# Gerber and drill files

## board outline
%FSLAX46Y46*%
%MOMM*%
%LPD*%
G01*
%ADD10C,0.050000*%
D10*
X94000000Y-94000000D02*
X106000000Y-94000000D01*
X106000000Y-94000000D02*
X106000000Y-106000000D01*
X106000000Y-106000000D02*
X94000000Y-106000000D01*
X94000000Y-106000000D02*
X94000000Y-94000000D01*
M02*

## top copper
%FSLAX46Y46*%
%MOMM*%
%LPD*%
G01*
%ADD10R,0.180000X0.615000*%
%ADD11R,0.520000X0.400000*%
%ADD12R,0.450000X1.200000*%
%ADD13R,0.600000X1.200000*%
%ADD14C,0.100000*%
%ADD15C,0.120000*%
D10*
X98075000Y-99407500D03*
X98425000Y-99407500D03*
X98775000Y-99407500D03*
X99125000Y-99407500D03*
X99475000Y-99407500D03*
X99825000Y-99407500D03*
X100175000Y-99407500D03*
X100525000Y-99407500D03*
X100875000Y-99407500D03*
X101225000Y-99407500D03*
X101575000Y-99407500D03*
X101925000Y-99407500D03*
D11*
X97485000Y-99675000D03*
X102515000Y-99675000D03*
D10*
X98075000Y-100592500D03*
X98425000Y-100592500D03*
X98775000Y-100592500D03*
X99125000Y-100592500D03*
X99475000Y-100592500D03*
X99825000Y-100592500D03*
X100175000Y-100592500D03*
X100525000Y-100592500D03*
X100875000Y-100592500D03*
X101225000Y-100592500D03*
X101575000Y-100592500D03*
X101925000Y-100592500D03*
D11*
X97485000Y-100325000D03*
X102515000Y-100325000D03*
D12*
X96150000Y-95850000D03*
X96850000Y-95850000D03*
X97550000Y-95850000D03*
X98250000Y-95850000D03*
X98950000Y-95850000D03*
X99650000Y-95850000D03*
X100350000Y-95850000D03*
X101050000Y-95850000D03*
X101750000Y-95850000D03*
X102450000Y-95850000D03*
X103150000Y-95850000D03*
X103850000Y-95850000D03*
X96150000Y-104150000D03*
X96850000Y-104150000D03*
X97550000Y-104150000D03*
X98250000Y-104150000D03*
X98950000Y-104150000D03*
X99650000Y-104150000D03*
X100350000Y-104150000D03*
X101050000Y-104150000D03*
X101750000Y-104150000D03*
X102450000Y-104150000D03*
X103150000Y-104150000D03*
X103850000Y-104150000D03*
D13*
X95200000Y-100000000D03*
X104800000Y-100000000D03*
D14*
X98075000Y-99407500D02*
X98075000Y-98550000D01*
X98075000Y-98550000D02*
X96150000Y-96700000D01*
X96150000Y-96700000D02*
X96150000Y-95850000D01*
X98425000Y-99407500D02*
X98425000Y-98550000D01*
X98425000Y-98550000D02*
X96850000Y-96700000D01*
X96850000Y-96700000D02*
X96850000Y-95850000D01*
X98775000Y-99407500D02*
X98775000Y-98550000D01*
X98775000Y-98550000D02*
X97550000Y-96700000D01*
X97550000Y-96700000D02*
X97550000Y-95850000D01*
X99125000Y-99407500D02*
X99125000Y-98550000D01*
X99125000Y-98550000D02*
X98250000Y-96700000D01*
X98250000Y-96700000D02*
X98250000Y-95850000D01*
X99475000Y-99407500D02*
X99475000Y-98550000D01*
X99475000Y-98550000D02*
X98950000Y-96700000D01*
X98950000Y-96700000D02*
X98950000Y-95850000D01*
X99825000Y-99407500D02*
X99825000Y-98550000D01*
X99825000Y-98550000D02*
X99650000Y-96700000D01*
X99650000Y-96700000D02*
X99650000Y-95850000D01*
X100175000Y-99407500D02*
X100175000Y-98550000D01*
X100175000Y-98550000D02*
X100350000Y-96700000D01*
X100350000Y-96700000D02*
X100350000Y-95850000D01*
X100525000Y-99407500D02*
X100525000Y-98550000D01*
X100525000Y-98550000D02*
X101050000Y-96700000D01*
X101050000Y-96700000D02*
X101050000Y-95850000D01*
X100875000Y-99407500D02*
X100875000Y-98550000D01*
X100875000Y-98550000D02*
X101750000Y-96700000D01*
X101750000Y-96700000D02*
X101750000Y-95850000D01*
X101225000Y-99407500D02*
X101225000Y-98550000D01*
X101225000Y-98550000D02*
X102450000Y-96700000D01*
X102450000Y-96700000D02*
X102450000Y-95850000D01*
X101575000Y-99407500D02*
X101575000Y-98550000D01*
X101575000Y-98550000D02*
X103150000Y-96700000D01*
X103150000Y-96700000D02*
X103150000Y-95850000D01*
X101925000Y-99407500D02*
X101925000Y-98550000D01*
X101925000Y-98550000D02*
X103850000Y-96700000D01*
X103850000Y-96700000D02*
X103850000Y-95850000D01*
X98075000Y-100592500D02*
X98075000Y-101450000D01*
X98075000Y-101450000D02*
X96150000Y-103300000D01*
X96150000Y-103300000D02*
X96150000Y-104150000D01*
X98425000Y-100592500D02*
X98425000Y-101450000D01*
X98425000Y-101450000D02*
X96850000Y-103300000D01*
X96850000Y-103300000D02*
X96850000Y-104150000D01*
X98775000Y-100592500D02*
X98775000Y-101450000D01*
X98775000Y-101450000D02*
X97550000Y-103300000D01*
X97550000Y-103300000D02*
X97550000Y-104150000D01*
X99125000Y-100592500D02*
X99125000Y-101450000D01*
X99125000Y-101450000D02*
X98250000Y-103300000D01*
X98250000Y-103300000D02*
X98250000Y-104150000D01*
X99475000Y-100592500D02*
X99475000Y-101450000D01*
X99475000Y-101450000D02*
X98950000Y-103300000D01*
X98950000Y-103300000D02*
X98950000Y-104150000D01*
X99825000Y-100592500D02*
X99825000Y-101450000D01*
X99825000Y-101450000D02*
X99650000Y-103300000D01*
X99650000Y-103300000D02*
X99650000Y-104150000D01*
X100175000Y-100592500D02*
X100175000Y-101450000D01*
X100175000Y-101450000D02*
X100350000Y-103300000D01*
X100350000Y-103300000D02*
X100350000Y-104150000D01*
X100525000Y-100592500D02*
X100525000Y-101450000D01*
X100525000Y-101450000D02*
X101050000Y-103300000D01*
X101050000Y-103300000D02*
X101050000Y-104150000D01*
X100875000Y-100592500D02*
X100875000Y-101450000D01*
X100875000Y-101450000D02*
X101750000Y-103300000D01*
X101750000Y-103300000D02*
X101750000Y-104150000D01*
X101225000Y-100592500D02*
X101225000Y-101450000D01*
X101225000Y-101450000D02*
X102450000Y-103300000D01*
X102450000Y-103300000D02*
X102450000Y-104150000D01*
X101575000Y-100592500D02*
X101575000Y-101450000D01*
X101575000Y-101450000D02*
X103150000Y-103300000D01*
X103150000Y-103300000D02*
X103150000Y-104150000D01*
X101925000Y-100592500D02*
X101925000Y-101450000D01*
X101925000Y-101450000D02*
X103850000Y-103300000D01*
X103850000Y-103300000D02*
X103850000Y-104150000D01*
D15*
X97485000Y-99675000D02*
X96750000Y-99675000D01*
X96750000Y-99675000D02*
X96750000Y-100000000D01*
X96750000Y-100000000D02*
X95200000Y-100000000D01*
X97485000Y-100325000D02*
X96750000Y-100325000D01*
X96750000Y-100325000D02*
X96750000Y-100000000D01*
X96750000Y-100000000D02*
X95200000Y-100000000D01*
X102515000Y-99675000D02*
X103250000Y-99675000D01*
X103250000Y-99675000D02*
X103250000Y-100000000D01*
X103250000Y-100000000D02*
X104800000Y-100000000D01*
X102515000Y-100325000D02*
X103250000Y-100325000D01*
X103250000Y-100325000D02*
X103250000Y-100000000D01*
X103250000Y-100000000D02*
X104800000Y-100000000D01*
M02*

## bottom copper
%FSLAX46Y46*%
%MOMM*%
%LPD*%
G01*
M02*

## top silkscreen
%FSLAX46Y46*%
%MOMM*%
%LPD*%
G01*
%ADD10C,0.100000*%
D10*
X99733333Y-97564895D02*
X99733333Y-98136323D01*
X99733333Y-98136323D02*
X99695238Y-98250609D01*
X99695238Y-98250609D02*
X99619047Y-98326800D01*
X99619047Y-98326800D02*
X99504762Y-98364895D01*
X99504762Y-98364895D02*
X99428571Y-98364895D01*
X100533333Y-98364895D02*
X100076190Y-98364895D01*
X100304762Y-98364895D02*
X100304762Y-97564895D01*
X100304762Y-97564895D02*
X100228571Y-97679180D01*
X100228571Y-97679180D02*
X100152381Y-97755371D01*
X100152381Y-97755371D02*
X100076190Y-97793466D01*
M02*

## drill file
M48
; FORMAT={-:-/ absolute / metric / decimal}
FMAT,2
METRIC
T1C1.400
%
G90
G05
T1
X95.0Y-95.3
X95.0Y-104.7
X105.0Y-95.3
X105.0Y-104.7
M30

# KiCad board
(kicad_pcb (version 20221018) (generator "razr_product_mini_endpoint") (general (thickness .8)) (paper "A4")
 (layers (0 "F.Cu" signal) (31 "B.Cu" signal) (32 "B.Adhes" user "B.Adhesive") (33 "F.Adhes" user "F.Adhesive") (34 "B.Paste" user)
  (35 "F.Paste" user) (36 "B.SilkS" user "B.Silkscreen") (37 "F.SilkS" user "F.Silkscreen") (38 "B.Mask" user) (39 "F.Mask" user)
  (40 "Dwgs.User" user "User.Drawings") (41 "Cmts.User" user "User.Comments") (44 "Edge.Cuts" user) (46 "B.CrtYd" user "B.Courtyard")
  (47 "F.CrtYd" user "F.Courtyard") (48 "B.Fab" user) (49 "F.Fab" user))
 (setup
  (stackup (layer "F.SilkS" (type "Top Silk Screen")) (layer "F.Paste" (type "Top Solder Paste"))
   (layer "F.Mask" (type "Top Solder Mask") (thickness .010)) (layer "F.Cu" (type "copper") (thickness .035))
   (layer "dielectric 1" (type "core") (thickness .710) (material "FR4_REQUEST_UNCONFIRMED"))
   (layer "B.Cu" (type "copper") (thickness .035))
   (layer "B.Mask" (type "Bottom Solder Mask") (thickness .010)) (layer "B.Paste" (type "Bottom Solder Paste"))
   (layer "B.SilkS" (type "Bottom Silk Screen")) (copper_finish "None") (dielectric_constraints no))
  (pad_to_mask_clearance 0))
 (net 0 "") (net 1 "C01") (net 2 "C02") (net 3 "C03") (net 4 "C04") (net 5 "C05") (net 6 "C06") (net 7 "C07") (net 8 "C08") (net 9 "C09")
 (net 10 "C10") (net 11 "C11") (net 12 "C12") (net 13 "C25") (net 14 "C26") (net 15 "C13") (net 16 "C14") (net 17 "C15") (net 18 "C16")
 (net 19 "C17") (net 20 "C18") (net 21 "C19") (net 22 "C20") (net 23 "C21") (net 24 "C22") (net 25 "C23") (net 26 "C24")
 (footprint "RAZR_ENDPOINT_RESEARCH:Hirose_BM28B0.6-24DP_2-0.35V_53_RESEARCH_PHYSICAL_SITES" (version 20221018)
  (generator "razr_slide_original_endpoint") (layer "F.Cu") (at 100 100)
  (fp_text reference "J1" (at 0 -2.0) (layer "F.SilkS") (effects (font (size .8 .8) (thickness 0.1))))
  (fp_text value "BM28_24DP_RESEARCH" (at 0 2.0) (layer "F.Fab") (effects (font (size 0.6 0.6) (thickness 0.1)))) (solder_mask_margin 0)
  (pad "S_NEG_00" smd rect (at -1.925 -0.5925) (size 0.18 0.615) (layers "F.Cu" "F.Mask") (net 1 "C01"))
  (pad "S_NEG_01" smd rect (at -1.575 -0.5925) (size 0.18 0.615) (layers "F.Cu" "F.Mask") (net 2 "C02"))
  (pad "S_NEG_02" smd rect (at -1.225 -0.5925) (size 0.18 0.615) (layers "F.Cu" "F.Mask") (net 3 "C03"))
  (pad "S_NEG_03" smd rect (at -0.875 -0.5925) (size 0.18 0.615) (layers "F.Cu" "F.Mask") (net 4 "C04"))
  (pad "S_NEG_04" smd rect (at -0.525 -0.5925) (size 0.18 0.615) (layers "F.Cu" "F.Mask") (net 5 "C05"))
  (pad "S_NEG_05" smd rect (at -0.175 -0.5925) (size 0.18 0.615) (layers "F.Cu" "F.Mask") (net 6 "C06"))
  (pad "S_NEG_06" smd rect (at 0.175 -0.5925) (size 0.18 0.615) (layers "F.Cu" "F.Mask") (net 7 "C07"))
  (pad "S_NEG_07" smd rect (at 0.525 -0.5925) (size 0.18 0.615) (layers "F.Cu" "F.Mask") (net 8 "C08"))
  (pad "S_NEG_08" smd rect (at 0.875 -0.5925) (size 0.18 0.615) (layers "F.Cu" "F.Mask") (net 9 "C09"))
  (pad "S_NEG_09" smd rect (at 1.225 -0.5925) (size 0.18 0.615) (layers "F.Cu" "F.Mask") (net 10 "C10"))
  (pad "S_NEG_10" smd rect (at 1.575 -0.5925) (size 0.18 0.615) (layers "F.Cu" "F.Mask") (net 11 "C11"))
  (pad "S_NEG_11" smd rect (at 1.925 -0.5925) (size 0.18 0.615) (layers "F.Cu" "F.Mask") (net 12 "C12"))
  (pad "P_L" smd rect (at -2.515 -0.325) (size 0.52 0.4) (layers "F.Cu" "F.Mask") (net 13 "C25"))
  (pad "P_R" smd rect (at 2.515 -0.325) (size 0.52 0.4) (layers "F.Cu" "F.Mask") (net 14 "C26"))
  (pad "S_POS_00" smd rect (at -1.925 0.5925) (size 0.18 0.615) (layers "F.Cu" "F.Mask") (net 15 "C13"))
  (pad "S_POS_01" smd rect (at -1.575 0.5925) (size 0.18 0.615) (layers "F.Cu" "F.Mask") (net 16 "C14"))
  (pad "S_POS_02" smd rect (at -1.225 0.5925) (size 0.18 0.615) (layers "F.Cu" "F.Mask") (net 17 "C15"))
  (pad "S_POS_03" smd rect (at -0.875 0.5925) (size 0.18 0.615) (layers "F.Cu" "F.Mask") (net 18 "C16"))
  (pad "S_POS_04" smd rect (at -0.525 0.5925) (size 0.18 0.615) (layers "F.Cu" "F.Mask") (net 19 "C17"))
  (pad "S_POS_05" smd rect (at -0.175 0.5925) (size 0.18 0.615) (layers "F.Cu" "F.Mask") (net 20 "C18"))
  (pad "S_POS_06" smd rect (at 0.175 0.5925) (size 0.18 0.615) (layers "F.Cu" "F.Mask") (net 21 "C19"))
  (pad "S_POS_07" smd rect (at 0.525 0.5925) (size 0.18 0.615) (layers "F.Cu" "F.Mask") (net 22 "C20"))
  (pad "S_POS_08" smd rect (at 0.875 0.5925) (size 0.18 0.615) (layers "F.Cu" "F.Mask") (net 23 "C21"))
  (pad "S_POS_09" smd rect (at 1.225 0.5925) (size 0.18 0.615) (layers "F.Cu" "F.Mask") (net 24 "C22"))
  (pad "S_POS_10" smd rect (at 1.575 0.5925) (size 0.18 0.615) (layers "F.Cu" "F.Mask") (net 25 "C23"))
  (pad "S_POS_11" smd rect (at 1.925 0.5925) (size 0.18 0.615) (layers "F.Cu" "F.Mask") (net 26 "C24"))
  (pad "P_L" smd rect (at -2.515 0.325) (size 0.52 0.4) (layers "F.Cu" "F.Mask") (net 13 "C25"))
  (pad "P_R" smd rect (at 2.515 0.325) (size 0.52 0.4) (layers "F.Cu" "F.Mask") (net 14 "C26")))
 (segment (start 98.075000 99.407500) (end 98.075000 98.550000) (width 0.1) (layer "F.Cu") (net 1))
 (segment (start 98.075000 98.550000) (end 96.150000 96.700000) (width 0.1) (layer "F.Cu") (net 1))
 (segment (start 96.150000 96.700000) (end 96.150000 95.850000) (width 0.1) (layer "F.Cu") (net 1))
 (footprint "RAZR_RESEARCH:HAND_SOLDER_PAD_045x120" (layer "F.Cu") (at 96.150000 95.850000)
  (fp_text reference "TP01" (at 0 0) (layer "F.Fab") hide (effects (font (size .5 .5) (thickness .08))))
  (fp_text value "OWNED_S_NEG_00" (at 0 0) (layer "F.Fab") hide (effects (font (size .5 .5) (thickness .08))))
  (pad "1" smd rect (at 0 0) (size 0.45 1.2) (layers "F.Cu" "F.Mask") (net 1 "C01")))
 (segment (start 98.425000 99.407500) (end 98.425000 98.550000) (width 0.1) (layer "F.Cu") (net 2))
 (segment (start 98.425000 98.550000) (end 96.850000 96.700000) (width 0.1) (layer "F.Cu") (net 2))
 (segment (start 96.850000 96.700000) (end 96.850000 95.850000) (width 0.1) (layer "F.Cu") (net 2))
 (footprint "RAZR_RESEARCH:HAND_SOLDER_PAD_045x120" (layer "F.Cu") (at 96.850000 95.850000)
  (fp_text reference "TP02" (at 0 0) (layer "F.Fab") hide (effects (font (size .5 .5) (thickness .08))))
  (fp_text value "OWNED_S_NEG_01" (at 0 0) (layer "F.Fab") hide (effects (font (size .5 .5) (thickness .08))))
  (pad "1" smd rect (at 0 0) (size 0.45 1.2) (layers "F.Cu" "F.Mask") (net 2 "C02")))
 (segment (start 98.775000 99.407500) (end 98.775000 98.550000) (width 0.1) (layer "F.Cu") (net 3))
 (segment (start 98.775000 98.550000) (end 97.550000 96.700000) (width 0.1) (layer "F.Cu") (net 3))
 (segment (start 97.550000 96.700000) (end 97.550000 95.850000) (width 0.1) (layer "F.Cu") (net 3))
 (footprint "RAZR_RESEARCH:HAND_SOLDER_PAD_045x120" (layer "F.Cu") (at 97.550000 95.850000)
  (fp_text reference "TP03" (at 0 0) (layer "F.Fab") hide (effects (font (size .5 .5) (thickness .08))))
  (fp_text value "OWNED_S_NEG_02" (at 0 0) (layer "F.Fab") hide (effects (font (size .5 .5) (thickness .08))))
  (pad "1" smd rect (at 0 0) (size 0.45 1.2) (layers "F.Cu" "F.Mask") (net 3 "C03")))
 (segment (start 99.125000 99.407500) (end 99.125000 98.550000) (width 0.1) (layer "F.Cu") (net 4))
 (segment (start 99.125000 98.550000) (end 98.250000 96.700000) (width 0.1) (layer "F.Cu") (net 4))
 (segment (start 98.250000 96.700000) (end 98.250000 95.850000) (width 0.1) (layer "F.Cu") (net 4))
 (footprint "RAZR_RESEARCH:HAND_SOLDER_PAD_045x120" (layer "F.Cu") (at 98.250000 95.850000)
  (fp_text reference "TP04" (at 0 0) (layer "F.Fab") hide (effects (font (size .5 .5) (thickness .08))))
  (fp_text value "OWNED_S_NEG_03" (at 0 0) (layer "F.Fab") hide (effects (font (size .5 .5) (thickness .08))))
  (pad "1" smd rect (at 0 0) (size 0.45 1.2) (layers "F.Cu" "F.Mask") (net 4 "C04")))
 (segment (start 99.475000 99.407500) (end 99.475000 98.550000) (width 0.1) (layer "F.Cu") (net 5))
 (segment (start 99.475000 98.550000) (end 98.950000 96.700000) (width 0.1) (layer "F.Cu") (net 5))
 (segment (start 98.950000 96.700000) (end 98.950000 95.850000) (width 0.1) (layer "F.Cu") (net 5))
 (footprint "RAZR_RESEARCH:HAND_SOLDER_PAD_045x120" (layer "F.Cu") (at 98.950000 95.850000)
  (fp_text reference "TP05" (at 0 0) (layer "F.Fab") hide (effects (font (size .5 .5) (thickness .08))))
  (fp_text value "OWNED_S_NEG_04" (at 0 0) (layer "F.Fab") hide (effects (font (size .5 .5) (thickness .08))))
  (pad "1" smd rect (at 0 0) (size 0.45 1.2) (layers "F.Cu" "F.Mask") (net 5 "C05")))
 (segment (start 99.825000 99.407500) (end 99.825000 98.550000) (width 0.1) (layer "F.Cu") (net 6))
 (segment (start 99.825000 98.550000) (end 99.650000 96.700000) (width 0.1) (layer "F.Cu") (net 6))
 (segment (start 99.650000 96.700000) (end 99.650000 95.850000) (width 0.1) (layer "F.Cu") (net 6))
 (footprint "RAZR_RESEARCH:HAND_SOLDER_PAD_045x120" (layer "F.Cu") (at 99.650000 95.850000)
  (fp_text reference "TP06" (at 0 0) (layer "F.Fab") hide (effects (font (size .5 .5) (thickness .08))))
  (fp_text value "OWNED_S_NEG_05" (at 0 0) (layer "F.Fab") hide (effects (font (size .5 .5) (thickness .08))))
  (pad "1" smd rect (at 0 0) (size 0.45 1.2) (layers "F.Cu" "F.Mask") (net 6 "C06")))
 (segment (start 100.175000 99.407500) (end 100.175000 98.550000) (width 0.1) (layer "F.Cu") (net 7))
 (segment (start 100.175000 98.550000) (end 100.350000 96.700000) (width 0.1) (layer "F.Cu") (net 7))
 (segment (start 100.350000 96.700000) (end 100.350000 95.850000) (width 0.1) (layer "F.Cu") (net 7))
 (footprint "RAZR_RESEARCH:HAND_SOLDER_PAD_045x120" (layer "F.Cu") (at 100.350000 95.850000)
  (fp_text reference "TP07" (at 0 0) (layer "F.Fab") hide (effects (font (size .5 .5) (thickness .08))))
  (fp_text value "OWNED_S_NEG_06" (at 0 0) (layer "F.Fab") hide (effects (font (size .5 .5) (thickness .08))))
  (pad "1" smd rect (at 0 0) (size 0.45 1.2) (layers "F.Cu" "F.Mask") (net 7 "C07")))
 (segment (start 100.525000 99.407500) (end 100.525000 98.550000) (width 0.1) (layer "F.Cu") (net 8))
 (segment (start 100.525000 98.550000) (end 101.050000 96.700000) (width 0.1) (layer "F.Cu") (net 8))
 (segment (start 101.050000 96.700000) (end 101.050000 95.850000) (width 0.1) (layer "F.Cu") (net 8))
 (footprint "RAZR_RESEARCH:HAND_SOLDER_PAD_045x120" (layer "F.Cu") (at 101.050000 95.850000)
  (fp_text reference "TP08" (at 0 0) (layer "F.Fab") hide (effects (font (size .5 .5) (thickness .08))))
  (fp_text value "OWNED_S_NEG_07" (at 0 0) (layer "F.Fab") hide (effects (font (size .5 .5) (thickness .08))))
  (pad "1" smd rect (at 0 0) (size 0.45 1.2) (layers "F.Cu" "F.Mask") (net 8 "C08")))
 (segment (start 100.875000 99.407500) (end 100.875000 98.550000) (width 0.1) (layer "F.Cu") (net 9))
 (segment (start 100.875000 98.550000) (end 101.750000 96.700000) (width 0.1) (layer "F.Cu") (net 9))
 (segment (start 101.750000 96.700000) (end 101.750000 95.850000) (width 0.1) (layer "F.Cu") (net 9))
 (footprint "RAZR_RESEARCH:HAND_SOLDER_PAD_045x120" (layer "F.Cu") (at 101.750000 95.850000)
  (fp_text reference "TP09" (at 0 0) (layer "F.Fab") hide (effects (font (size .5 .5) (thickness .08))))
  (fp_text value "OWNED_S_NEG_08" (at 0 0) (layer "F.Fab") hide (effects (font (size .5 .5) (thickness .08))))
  (pad "1" smd rect (at 0 0) (size 0.45 1.2) (layers "F.Cu" "F.Mask") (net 9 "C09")))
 (segment (start 101.225000 99.407500) (end 101.225000 98.550000) (width 0.1) (layer "F.Cu") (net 10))
 (segment (start 101.225000 98.550000) (end 102.450000 96.700000) (width 0.1) (layer "F.Cu") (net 10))
 (segment (start 102.450000 96.700000) (end 102.450000 95.850000) (width 0.1) (layer "F.Cu") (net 10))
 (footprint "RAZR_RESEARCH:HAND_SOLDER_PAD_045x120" (layer "F.Cu") (at 102.450000 95.850000)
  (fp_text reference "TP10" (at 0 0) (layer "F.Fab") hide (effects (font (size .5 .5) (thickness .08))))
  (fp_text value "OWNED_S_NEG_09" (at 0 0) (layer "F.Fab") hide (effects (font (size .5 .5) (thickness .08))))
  (pad "1" smd rect (at 0 0) (size 0.45 1.2) (layers "F.Cu" "F.Mask") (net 10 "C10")))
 (segment (start 101.575000 99.407500) (end 101.575000 98.550000) (width 0.1) (layer "F.Cu") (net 11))
 (segment (start 101.575000 98.550000) (end 103.150000 96.700000) (width 0.1) (layer "F.Cu") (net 11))
 (segment (start 103.150000 96.700000) (end 103.150000 95.850000) (width 0.1) (layer "F.Cu") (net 11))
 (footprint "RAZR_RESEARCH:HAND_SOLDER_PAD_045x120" (layer "F.Cu") (at 103.150000 95.850000)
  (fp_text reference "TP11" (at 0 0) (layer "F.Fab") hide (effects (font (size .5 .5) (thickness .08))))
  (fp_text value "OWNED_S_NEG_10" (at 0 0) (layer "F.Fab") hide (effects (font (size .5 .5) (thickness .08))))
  (pad "1" smd rect (at 0 0) (size 0.45 1.2) (layers "F.Cu" "F.Mask") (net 11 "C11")))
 (segment (start 101.925000 99.407500) (end 101.925000 98.550000) (width 0.1) (layer "F.Cu") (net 12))
 (segment (start 101.925000 98.550000) (end 103.850000 96.700000) (width 0.1) (layer "F.Cu") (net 12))
 (segment (start 103.850000 96.700000) (end 103.850000 95.850000) (width 0.1) (layer "F.Cu") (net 12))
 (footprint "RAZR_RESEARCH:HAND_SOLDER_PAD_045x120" (layer "F.Cu") (at 103.850000 95.850000)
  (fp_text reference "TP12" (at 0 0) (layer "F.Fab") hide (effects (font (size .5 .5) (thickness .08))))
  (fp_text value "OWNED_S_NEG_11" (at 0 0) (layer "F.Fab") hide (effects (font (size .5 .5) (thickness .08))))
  (pad "1" smd rect (at 0 0) (size 0.45 1.2) (layers "F.Cu" "F.Mask") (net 12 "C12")))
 (segment (start 98.075000 100.592500) (end 98.075000 101.450000) (width 0.1) (layer "F.Cu") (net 15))
 (segment (start 98.075000 101.450000) (end 96.150000 103.300000) (width 0.1) (layer "F.Cu") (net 15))
 (segment (start 96.150000 103.300000) (end 96.150000 104.150000) (width 0.1) (layer "F.Cu") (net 15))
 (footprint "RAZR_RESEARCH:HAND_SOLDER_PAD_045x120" (layer "F.Cu") (at 96.150000 104.150000)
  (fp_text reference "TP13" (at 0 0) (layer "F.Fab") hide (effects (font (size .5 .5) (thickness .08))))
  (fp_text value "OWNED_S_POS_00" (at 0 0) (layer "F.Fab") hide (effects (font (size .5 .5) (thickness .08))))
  (pad "1" smd rect (at 0 0) (size 0.45 1.2) (layers "F.Cu" "F.Mask") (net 15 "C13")))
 (segment (start 98.425000 100.592500) (end 98.425000 101.450000) (width 0.1) (layer "F.Cu") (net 16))
 (segment (start 98.425000 101.450000) (end 96.850000 103.300000) (width 0.1) (layer "F.Cu") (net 16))
 (segment (start 96.850000 103.300000) (end 96.850000 104.150000) (width 0.1) (layer "F.Cu") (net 16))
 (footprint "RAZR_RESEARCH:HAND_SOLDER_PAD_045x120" (layer "F.Cu") (at 96.850000 104.150000)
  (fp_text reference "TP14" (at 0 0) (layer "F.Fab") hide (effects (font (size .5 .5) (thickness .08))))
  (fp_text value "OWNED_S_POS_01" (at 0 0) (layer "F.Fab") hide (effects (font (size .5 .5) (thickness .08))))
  (pad "1" smd rect (at 0 0) (size 0.45 1.2) (layers "F.Cu" "F.Mask") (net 16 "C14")))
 (segment (start 98.775000 100.592500) (end 98.775000 101.450000) (width 0.1) (layer "F.Cu") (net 17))
 (segment (start 98.775000 101.450000) (end 97.550000 103.300000) (width 0.1) (layer "F.Cu") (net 17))
 (segment (start 97.550000 103.300000) (end 97.550000 104.150000) (width 0.1) (layer "F.Cu") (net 17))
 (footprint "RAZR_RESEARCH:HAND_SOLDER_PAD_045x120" (layer "F.Cu") (at 97.550000 104.150000)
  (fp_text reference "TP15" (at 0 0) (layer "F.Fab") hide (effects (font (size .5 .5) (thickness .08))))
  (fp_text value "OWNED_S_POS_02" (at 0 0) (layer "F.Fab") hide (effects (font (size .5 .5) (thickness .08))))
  (pad "1" smd rect (at 0 0) (size 0.45 1.2) (layers "F.Cu" "F.Mask") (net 17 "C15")))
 (segment (start 99.125000 100.592500) (end 99.125000 101.450000) (width 0.1) (layer "F.Cu") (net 18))
 (segment (start 99.125000 101.450000) (end 98.250000 103.300000) (width 0.1) (layer "F.Cu") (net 18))
 (segment (start 98.250000 103.300000) (end 98.250000 104.150000) (width 0.1) (layer "F.Cu") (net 18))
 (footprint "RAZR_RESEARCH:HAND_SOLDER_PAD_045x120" (layer "F.Cu") (at 98.250000 104.150000)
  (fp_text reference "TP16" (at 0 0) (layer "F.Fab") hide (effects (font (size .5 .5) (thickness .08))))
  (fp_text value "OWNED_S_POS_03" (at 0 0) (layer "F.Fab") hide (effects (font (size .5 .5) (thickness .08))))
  (pad "1" smd rect (at 0 0) (size 0.45 1.2) (layers "F.Cu" "F.Mask") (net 18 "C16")))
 (segment (start 99.475000 100.592500) (end 99.475000 101.450000) (width 0.1) (layer "F.Cu") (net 19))
 (segment (start 99.475000 101.450000) (end 98.950000 103.300000) (width 0.1) (layer "F.Cu") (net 19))
 (segment (start 98.950000 103.300000) (end 98.950000 104.150000) (width 0.1) (layer "F.Cu") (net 19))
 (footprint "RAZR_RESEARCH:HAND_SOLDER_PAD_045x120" (layer "F.Cu") (at 98.950000 104.150000)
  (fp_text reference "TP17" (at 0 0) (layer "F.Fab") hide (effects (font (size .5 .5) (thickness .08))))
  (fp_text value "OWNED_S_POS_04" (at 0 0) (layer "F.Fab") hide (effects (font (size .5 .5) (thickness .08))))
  (pad "1" smd rect (at 0 0) (size 0.45 1.2) (layers "F.Cu" "F.Mask") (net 19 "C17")))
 (segment (start 99.825000 100.592500) (end 99.825000 101.450000) (width 0.1) (layer "F.Cu") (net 20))
 (segment (start 99.825000 101.450000) (end 99.650000 103.300000) (width 0.1) (layer "F.Cu") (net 20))
 (segment (start 99.650000 103.300000) (end 99.650000 104.150000) (width 0.1) (layer "F.Cu") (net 20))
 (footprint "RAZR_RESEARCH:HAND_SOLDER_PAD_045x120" (layer "F.Cu") (at 99.650000 104.150000)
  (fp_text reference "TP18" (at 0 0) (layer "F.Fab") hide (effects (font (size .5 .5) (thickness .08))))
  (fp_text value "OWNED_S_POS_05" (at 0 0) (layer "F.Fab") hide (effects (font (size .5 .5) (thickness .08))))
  (pad "1" smd rect (at 0 0) (size 0.45 1.2) (layers "F.Cu" "F.Mask") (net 20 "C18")))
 (segment (start 100.175000 100.592500) (end 100.175000 101.450000) (width 0.1) (layer "F.Cu") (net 21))
 (segment (start 100.175000 101.450000) (end 100.350000 103.300000) (width 0.1) (layer "F.Cu") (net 21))
 (segment (start 100.350000 103.300000) (end 100.350000 104.150000) (width 0.1) (layer "F.Cu") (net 21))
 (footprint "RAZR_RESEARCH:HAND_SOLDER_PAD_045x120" (layer "F.Cu") (at 100.350000 104.150000)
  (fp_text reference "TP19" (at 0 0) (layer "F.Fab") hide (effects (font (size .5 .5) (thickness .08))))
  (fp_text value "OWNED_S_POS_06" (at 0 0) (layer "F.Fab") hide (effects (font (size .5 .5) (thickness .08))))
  (pad "1" smd rect (at 0 0) (size 0.45 1.2) (layers "F.Cu" "F.Mask") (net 21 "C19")))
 (segment (start 100.525000 100.592500) (end 100.525000 101.450000) (width 0.1) (layer "F.Cu") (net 22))
 (segment (start 100.525000 101.450000) (end 101.050000 103.300000) (width 0.1) (layer "F.Cu") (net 22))
 (segment (start 101.050000 103.300000) (end 101.050000 104.150000) (width 0.1) (layer "F.Cu") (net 22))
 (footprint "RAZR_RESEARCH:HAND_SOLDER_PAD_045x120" (layer "F.Cu") (at 101.050000 104.150000)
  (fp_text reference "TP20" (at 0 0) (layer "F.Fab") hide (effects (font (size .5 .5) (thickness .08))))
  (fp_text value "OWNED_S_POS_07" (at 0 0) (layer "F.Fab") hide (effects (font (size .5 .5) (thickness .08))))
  (pad "1" smd rect (at 0 0) (size 0.45 1.2) (layers "F.Cu" "F.Mask") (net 22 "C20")))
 (segment (start 100.875000 100.592500) (end 100.875000 101.450000) (width 0.1) (layer "F.Cu") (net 23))
 (segment (start 100.875000 101.450000) (end 101.750000 103.300000) (width 0.1) (layer "F.Cu") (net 23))
 (segment (start 101.750000 103.300000) (end 101.750000 104.150000) (width 0.1) (layer "F.Cu") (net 23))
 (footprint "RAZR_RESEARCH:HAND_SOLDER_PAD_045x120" (layer "F.Cu") (at 101.750000 104.150000)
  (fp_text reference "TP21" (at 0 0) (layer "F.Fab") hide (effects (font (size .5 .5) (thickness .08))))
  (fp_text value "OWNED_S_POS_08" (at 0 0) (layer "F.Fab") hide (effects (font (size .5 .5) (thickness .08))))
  (pad "1" smd rect (at 0 0) (size 0.45 1.2) (layers "F.Cu" "F.Mask") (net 23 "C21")))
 (segment (start 101.225000 100.592500) (end 101.225000 101.450000) (width 0.1) (layer "F.Cu") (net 24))
 (segment (start 101.225000 101.450000) (end 102.450000 103.300000) (width 0.1) (layer "F.Cu") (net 24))
 (segment (start 102.450000 103.300000) (end 102.450000 104.150000) (width 0.1) (layer "F.Cu") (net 24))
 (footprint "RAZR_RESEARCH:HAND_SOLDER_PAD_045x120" (layer "F.Cu") (at 102.450000 104.150000)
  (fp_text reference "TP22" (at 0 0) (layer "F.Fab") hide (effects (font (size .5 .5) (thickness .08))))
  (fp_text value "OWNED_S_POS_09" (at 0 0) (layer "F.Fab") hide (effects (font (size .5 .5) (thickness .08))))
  (pad "1" smd rect (at 0 0) (size 0.45 1.2) (layers "F.Cu" "F.Mask") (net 24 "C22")))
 (segment (start 101.575000 100.592500) (end 101.575000 101.450000) (width 0.1) (layer "F.Cu") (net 25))
 (segment (start 101.575000 101.450000) (end 103.150000 103.300000) (width 0.1) (layer "F.Cu") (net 25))
 (segment (start 103.150000 103.300000) (end 103.150000 104.150000) (width 0.1) (layer "F.Cu") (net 25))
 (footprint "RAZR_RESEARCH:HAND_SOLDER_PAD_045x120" (layer "F.Cu") (at 103.150000 104.150000)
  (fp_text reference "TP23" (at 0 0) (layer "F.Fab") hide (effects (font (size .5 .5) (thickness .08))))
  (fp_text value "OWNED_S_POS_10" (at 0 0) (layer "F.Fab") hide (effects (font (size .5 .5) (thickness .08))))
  (pad "1" smd rect (at 0 0) (size 0.45 1.2) (layers "F.Cu" "F.Mask") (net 25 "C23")))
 (segment (start 101.925000 100.592500) (end 101.925000 101.450000) (width 0.1) (layer "F.Cu") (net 26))
 (segment (start 101.925000 101.450000) (end 103.850000 103.300000) (width 0.1) (layer "F.Cu") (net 26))
 (segment (start 103.850000 103.300000) (end 103.850000 104.150000) (width 0.1) (layer "F.Cu") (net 26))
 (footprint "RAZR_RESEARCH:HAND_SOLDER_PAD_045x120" (layer "F.Cu") (at 103.850000 104.150000)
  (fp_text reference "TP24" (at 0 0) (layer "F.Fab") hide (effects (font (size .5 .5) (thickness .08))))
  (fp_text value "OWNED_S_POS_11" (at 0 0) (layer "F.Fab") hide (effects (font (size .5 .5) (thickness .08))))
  (pad "1" smd rect (at 0 0) (size 0.45 1.2) (layers "F.Cu" "F.Mask") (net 26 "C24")))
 (segment (start 97.485000 99.675000) (end 96.750000 99.675000) (width 0.12) (layer "F.Cu") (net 13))
 (segment (start 96.750000 99.675000) (end 96.750000 100.000000) (width 0.12) (layer "F.Cu") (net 13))
 (segment (start 96.750000 100.000000) (end 95.200000 100.000000) (width 0.12) (layer "F.Cu") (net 13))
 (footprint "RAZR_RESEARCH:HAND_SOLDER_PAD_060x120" (layer "F.Cu") (at 95.200000 100.000000)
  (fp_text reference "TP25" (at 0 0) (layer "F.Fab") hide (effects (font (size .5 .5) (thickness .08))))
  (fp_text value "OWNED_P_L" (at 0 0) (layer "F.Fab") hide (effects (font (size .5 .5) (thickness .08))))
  (pad "1" smd rect (at 0 0) (size 0.6 1.2) (layers "F.Cu" "F.Mask") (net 13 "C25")))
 (segment (start 97.485000 100.325000) (end 96.750000 100.325000) (width 0.12) (layer "F.Cu") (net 13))
 (segment (start 96.750000 100.325000) (end 96.750000 100.000000) (width 0.12) (layer "F.Cu") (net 13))
 (segment (start 96.750000 100.000000) (end 95.200000 100.000000) (width 0.12) (layer "F.Cu") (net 13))
 (segment (start 102.515000 99.675000) (end 103.250000 99.675000) (width 0.12) (layer "F.Cu") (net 14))
 (segment (start 103.250000 99.675000) (end 103.250000 100.000000) (width 0.12) (layer "F.Cu") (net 14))
 (segment (start 103.250000 100.000000) (end 104.800000 100.000000) (width 0.12) (layer "F.Cu") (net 14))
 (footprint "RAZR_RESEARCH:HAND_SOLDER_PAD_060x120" (layer "F.Cu") (at 104.800000 100.000000)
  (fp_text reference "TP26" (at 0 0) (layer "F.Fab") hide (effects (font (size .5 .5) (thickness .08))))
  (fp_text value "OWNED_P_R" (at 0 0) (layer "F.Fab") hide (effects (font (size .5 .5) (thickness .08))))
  (pad "1" smd rect (at 0 0) (size 0.6 1.2) (layers "F.Cu" "F.Mask") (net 14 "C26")))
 (segment (start 102.515000 100.325000) (end 103.250000 100.325000) (width 0.12) (layer "F.Cu") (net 14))
 (segment (start 103.250000 100.325000) (end 103.250000 100.000000) (width 0.12) (layer "F.Cu") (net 14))
 (segment (start 103.250000 100.000000) (end 104.800000 100.000000) (width 0.12) (layer "F.Cu") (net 14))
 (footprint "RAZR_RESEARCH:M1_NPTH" (layer "F.Cu") (at 95 95.3)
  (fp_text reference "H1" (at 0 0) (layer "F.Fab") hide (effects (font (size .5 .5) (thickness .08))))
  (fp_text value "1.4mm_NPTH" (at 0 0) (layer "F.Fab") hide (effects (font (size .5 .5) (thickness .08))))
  (pad "" np_thru_hole circle (at 0 0) (size 1.4 1.4) (drill 1.4) (layers "*.Cu" "*.Mask")))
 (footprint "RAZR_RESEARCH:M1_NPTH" (layer "F.Cu") (at 105 95.3)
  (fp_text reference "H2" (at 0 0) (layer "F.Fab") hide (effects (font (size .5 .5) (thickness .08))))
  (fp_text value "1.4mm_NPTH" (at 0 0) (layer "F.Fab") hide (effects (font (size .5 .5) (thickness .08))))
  (pad "" np_thru_hole circle (at 0 0) (size 1.4 1.4) (drill 1.4) (layers "*.Cu" "*.Mask")))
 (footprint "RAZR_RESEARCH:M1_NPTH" (layer "F.Cu") (at 95 104.7)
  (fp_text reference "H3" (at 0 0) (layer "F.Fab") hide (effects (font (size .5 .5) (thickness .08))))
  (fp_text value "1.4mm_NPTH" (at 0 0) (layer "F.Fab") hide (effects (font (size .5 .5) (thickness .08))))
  (pad "" np_thru_hole circle (at 0 0) (size 1.4 1.4) (drill 1.4) (layers "*.Cu" "*.Mask")))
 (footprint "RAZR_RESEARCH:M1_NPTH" (layer "F.Cu") (at 105 104.7)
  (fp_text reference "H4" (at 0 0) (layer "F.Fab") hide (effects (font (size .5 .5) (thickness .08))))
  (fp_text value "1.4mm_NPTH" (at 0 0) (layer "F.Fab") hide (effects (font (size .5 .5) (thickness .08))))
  (pad "" np_thru_hole circle (at 0 0) (size 1.4 1.4) (drill 1.4) (layers "*.Cu" "*.Mask")))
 (gr_line (start 94 94) (end 106 94) (layer "Edge.Cuts") (width .05))
 (gr_line (start 106 94) (end 106 106) (layer "Edge.Cuts") (width .05))
 (gr_line (start 106 106) (end 94 106) (layer "Edge.Cuts") (width .05))
 (gr_line (start 94 106) (end 94 94) (layer "Edge.Cuts") (width .05)))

